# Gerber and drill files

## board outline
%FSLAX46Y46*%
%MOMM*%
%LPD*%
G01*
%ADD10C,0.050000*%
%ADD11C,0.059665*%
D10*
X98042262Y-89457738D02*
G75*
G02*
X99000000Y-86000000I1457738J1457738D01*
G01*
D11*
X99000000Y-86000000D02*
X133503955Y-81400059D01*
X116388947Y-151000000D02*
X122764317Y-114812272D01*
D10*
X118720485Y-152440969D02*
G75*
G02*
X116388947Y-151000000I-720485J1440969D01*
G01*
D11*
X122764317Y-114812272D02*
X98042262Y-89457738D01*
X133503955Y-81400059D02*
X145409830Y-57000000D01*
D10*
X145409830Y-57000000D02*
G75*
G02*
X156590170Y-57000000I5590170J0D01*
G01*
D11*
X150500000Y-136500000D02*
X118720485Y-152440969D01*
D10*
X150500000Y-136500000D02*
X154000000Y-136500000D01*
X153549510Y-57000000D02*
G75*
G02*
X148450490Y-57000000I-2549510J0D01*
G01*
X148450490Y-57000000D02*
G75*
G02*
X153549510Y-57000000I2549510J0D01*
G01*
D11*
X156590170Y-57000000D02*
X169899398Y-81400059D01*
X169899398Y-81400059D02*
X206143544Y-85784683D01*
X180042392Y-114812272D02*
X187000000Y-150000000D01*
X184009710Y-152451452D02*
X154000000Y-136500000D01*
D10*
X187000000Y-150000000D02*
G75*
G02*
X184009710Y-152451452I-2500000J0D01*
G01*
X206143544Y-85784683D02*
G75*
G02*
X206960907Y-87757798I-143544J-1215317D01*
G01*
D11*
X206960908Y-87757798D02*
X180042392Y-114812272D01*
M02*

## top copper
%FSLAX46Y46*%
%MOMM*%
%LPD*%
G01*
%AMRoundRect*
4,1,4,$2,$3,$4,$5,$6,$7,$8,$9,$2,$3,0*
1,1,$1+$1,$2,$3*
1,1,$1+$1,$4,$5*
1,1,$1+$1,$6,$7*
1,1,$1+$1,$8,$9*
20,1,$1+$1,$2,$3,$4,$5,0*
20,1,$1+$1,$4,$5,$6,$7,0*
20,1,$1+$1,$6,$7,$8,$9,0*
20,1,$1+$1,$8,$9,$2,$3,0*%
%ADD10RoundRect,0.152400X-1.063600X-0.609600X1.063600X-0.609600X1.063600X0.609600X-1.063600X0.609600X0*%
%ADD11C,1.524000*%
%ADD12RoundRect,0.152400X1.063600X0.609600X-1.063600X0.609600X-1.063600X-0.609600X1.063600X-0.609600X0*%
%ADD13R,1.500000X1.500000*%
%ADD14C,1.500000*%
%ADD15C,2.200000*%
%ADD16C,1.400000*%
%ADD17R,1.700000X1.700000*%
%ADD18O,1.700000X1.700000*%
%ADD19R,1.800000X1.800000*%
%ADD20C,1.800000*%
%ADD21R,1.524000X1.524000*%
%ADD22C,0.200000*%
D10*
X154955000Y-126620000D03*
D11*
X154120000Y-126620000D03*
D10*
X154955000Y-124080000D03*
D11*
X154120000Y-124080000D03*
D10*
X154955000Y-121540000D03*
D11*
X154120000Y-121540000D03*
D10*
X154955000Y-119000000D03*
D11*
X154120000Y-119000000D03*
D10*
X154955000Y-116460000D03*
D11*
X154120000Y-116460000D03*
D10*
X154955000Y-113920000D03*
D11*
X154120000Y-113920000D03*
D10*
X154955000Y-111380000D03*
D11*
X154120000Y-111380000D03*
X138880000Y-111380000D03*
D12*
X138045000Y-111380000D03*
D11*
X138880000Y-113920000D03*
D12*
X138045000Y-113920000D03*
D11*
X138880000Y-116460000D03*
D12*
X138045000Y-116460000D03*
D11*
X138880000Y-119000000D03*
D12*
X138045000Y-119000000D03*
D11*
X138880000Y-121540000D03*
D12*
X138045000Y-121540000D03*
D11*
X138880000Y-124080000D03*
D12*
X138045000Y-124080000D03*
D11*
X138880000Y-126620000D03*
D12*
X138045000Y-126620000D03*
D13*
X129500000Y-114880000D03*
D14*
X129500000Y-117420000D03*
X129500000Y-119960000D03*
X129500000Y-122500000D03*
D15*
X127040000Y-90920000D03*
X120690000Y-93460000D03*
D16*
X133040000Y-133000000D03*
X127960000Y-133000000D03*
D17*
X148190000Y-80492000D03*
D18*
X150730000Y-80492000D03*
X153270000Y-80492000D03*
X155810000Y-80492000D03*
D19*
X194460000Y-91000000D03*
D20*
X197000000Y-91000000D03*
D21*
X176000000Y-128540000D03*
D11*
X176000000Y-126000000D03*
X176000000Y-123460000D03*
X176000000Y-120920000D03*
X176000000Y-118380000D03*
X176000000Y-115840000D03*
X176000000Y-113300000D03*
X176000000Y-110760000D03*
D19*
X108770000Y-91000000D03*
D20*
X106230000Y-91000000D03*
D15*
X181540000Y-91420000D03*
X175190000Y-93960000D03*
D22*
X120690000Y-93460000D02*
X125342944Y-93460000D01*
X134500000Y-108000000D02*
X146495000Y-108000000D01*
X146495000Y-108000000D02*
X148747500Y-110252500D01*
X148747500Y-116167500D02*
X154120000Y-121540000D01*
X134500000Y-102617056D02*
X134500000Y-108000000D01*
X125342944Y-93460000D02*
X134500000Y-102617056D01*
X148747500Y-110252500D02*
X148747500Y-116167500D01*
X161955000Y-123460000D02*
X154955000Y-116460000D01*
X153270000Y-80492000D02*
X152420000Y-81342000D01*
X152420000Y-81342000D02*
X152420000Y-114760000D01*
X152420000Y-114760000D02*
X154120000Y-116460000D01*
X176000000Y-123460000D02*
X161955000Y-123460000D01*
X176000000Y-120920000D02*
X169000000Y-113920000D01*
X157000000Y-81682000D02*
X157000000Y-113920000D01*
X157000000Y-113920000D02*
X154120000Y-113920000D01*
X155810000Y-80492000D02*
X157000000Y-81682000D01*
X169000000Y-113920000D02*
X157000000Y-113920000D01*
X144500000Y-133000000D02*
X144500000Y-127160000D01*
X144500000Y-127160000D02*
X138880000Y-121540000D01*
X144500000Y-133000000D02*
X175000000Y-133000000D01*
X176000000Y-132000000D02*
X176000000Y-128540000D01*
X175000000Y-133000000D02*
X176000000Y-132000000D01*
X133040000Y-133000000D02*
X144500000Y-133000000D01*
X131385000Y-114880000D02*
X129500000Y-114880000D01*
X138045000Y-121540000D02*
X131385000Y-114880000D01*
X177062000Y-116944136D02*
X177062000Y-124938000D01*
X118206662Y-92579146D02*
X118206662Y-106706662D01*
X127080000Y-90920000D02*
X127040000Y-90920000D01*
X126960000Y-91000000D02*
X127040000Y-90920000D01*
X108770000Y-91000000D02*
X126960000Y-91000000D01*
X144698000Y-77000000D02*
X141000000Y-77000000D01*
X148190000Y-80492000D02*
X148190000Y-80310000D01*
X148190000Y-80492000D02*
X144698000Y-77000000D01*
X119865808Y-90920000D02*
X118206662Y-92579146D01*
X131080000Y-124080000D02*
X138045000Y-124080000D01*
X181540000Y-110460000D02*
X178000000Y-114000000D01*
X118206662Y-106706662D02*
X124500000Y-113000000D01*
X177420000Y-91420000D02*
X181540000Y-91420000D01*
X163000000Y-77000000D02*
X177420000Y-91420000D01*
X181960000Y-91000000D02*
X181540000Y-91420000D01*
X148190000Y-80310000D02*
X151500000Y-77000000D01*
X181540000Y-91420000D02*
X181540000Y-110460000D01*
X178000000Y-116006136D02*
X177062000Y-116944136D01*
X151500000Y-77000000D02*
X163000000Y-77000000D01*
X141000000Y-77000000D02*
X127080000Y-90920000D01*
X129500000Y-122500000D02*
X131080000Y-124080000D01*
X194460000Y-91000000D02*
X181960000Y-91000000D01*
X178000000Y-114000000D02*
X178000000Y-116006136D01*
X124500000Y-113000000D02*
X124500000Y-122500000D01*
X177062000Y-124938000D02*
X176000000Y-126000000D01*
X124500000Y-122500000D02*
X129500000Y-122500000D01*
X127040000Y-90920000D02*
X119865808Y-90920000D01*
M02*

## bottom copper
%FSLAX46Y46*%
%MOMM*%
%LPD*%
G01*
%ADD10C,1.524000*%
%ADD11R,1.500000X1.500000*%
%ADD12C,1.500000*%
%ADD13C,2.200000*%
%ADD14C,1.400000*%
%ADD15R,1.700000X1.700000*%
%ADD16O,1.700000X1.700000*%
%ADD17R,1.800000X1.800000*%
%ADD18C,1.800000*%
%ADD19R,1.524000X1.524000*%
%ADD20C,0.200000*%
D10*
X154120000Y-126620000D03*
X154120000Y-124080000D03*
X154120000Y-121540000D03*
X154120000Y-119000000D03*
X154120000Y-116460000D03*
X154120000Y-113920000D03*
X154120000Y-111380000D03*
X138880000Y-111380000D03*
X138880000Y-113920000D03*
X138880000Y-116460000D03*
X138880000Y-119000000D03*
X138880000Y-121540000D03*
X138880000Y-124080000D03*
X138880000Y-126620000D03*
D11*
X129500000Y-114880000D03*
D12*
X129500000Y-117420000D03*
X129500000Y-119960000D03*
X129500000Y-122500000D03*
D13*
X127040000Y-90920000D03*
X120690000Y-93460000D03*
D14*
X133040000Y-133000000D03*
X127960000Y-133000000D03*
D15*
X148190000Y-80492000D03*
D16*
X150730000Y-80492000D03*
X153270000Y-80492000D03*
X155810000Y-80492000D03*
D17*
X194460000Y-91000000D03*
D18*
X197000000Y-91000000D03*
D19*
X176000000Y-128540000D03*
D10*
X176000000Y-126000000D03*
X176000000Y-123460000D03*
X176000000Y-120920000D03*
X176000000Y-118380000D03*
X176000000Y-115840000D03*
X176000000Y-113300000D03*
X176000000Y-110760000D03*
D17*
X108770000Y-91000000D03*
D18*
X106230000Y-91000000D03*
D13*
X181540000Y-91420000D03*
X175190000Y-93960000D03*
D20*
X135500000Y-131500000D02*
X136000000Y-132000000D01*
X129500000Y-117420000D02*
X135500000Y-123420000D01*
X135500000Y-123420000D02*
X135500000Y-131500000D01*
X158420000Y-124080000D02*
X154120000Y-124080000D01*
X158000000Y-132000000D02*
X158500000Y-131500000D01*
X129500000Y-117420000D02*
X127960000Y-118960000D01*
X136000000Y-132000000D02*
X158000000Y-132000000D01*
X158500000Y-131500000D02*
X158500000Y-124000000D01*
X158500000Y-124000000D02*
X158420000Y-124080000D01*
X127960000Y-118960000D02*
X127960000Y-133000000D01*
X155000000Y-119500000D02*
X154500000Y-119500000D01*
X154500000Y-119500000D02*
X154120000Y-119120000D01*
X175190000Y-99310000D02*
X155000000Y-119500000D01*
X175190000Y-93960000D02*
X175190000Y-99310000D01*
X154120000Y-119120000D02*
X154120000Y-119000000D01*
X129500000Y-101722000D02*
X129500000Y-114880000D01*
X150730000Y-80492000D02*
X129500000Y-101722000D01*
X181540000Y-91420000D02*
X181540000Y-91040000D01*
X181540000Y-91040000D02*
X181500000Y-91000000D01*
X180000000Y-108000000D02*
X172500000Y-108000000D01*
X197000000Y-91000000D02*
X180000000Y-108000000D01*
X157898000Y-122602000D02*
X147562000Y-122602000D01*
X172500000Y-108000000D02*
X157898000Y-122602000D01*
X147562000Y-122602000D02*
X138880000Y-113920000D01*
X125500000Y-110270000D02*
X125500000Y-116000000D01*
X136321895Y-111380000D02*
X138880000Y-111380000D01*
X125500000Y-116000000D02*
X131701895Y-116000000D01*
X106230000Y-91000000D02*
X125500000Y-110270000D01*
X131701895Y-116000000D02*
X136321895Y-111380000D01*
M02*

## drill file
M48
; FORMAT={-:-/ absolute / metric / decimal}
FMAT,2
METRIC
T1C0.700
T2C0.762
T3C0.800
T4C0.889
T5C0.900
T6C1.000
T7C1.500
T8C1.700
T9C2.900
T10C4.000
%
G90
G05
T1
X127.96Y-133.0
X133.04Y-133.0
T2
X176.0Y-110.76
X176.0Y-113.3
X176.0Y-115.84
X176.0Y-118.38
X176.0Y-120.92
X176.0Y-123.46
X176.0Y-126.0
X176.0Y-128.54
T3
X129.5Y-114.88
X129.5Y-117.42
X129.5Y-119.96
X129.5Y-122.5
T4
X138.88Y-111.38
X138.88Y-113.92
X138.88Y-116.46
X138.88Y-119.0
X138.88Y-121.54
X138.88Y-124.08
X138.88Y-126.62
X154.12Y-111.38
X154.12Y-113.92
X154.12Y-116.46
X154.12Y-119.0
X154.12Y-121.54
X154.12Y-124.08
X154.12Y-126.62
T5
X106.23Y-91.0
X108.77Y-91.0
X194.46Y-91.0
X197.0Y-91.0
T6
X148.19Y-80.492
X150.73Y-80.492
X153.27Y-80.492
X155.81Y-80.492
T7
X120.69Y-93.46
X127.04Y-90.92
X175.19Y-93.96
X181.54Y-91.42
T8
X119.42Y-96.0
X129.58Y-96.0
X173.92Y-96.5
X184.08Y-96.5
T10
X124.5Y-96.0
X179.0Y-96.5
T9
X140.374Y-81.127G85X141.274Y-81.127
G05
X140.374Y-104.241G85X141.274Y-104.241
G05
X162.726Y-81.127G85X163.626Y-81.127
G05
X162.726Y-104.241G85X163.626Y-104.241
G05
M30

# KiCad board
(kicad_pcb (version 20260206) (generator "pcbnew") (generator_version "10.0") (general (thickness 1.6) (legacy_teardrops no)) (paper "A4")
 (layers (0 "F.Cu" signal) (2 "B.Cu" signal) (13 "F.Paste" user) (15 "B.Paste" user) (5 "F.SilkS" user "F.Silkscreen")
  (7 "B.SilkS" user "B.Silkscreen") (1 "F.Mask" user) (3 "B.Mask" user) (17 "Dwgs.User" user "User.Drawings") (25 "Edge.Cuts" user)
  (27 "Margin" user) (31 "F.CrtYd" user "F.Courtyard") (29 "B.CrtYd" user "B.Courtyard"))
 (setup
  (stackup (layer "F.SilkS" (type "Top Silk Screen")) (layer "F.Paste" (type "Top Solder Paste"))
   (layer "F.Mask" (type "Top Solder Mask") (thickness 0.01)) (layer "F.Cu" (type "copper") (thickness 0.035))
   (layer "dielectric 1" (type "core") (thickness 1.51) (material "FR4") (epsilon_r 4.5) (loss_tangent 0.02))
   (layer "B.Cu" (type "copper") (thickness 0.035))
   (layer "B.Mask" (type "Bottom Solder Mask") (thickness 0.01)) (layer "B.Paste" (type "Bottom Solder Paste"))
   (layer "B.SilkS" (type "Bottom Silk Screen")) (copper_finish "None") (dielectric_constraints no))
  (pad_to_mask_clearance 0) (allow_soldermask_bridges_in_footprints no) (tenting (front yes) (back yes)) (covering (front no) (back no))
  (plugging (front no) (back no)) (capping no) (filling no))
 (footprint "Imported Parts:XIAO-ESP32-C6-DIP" (layer "F.Cu") (at 146.5 119 -90)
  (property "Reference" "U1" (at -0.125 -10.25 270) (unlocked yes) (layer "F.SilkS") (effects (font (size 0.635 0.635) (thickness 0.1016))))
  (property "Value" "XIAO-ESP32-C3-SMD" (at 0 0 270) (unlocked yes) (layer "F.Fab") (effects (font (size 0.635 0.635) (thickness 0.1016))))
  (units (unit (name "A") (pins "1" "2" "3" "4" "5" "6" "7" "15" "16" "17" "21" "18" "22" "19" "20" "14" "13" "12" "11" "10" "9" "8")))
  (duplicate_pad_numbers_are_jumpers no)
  (pad "1" smd roundrect (at 7.62 -8.455) (size 2.432 1.524) (layers "F.Cu" "F.Mask") (roundrect_rratio 0.1)
   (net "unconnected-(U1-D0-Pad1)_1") (thermal_bridge_angle 45))
  (pad "1" thru_hole circle (at 7.62 -7.62) (size 1.524 1.524) (drill 0.889) (layers "*.Cu" "*.Mask") (remove_unused_layers no)
   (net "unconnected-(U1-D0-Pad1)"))
  (pad "2" smd roundrect (at 5.08 -8.455) (size 2.432 1.524) (layers "F.Cu" "F.Mask") (roundrect_rratio 0.1) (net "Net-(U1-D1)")
   (thermal_bridge_angle 45))
  (pad "2" thru_hole circle (at 5.08 -7.62) (size 1.524 1.524) (drill 0.889) (layers "*.Cu" "*.Mask") (remove_unused_layers no)
   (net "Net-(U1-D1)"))
  (pad "3" smd roundrect (at 2.54 -8.455) (size 2.432 1.524) (layers "F.Cu" "F.Mask") (roundrect_rratio 0.1) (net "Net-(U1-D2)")
   (thermal_bridge_angle 45))
  (pad "3" thru_hole circle (at 2.54 -7.62) (size 1.524 1.524) (drill 0.889) (layers "*.Cu" "*.Mask") (remove_unused_layers no)
   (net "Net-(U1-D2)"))
  (pad "4" smd roundrect (at 0 -8.455) (size 2.432 1.524) (layers "F.Cu" "F.Mask") (roundrect_rratio 0.1) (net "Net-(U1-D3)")
   (thermal_bridge_angle 45))
  (pad "4" thru_hole circle (at 0 -7.62) (size 1.524 1.524) (drill 0.889) (layers "*.Cu" "*.Mask") (remove_unused_layers no)
   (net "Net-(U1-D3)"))
  (pad "5" smd roundrect (at -2.54 -8.455) (size 2.432 1.524) (layers "F.Cu" "F.Mask") (roundrect_rratio 0.1) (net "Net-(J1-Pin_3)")
   (thermal_bridge_angle 45))
  (pad "5" thru_hole circle (at -2.54 -7.62) (size 1.524 1.524) (drill 0.889) (layers "*.Cu" "*.Mask") (remove_unused_layers no)
   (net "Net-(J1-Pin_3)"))
  (pad "6" smd roundrect (at -5.08 -8.455) (size 2.432 1.524) (layers "F.Cu" "F.Mask") (roundrect_rratio 0.1) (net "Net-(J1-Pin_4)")
   (thermal_bridge_angle 45))
  (pad "6" thru_hole circle (at -5.08 -7.62) (size 1.524 1.524) (drill 0.889) (layers "*.Cu" "*.Mask") (remove_unused_layers no)
   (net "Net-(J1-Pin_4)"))
  (pad "7" smd roundrect (at -7.62 -8.455) (size 2.432 1.524) (layers "F.Cu" "F.Mask") (roundrect_rratio 0.1)
   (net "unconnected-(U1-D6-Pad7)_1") (thermal_bridge_angle 45))
  (pad "7" thru_hole circle (at -7.62 -7.62) (size 1.524 1.524) (drill 0.889) (layers "*.Cu" "*.Mask") (remove_unused_layers no)
   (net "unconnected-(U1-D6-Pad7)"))
  (pad "8" thru_hole circle (at -7.62 7.62 180) (size 1.524 1.524) (drill 0.889) (layers "*.Cu" "*.Mask") (remove_unused_layers no)
   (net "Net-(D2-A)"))
  (pad "8" smd roundrect (at -7.62 8.455 180) (size 2.432 1.524) (layers "F.Cu" "F.Mask") (roundrect_rratio 0.1) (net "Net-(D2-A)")
   (thermal_bridge_angle 45))
  (pad "9" thru_hole circle (at -5.08 7.62 180) (size 1.524 1.524) (drill 0.889) (layers "*.Cu" "*.Mask") (remove_unused_layers no)
   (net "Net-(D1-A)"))
  (pad "9" smd roundrect (at -5.08 8.455 180) (size 2.432 1.524) (layers "F.Cu" "F.Mask") (roundrect_rratio 0.1) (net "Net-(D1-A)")
   (thermal_bridge_angle 45))
  (pad "10" thru_hole circle (at -2.54 7.62 180) (size 1.524 1.524) (drill 0.889) (layers "*.Cu" "*.Mask") (remove_unused_layers no)
   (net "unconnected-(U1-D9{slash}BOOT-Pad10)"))
  (pad "10" smd roundrect (at -2.54 8.455 180) (size 2.432 1.524) (layers "F.Cu" "F.Mask") (roundrect_rratio 0.1)
   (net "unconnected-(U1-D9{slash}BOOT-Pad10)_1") (thermal_bridge_angle 45))
  (pad "11" thru_hole circle (at 0 7.62 180) (size 1.524 1.524) (drill 0.889) (layers "*.Cu" "*.Mask") (remove_unused_layers no)
   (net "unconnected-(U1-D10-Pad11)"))
  (pad "11" smd roundrect (at 0 8.455 180) (size 2.432 1.524) (layers "F.Cu" "F.Mask") (roundrect_rratio 0.1)
   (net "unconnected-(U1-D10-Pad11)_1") (thermal_bridge_angle 45))
  (pad "12" thru_hole circle (at 2.54 7.62 180) (size 1.524 1.524) (drill 0.889) (layers "*.Cu" "*.Mask") (remove_unused_layers no)
   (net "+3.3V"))
  (pad "12" smd roundrect (at 2.54 8.455 180) (size 2.432 1.524) (layers "F.Cu" "F.Mask") (roundrect_rratio 0.1) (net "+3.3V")
   (thermal_bridge_angle 45))
  (pad "13" thru_hole circle (at 5.08 7.62 180) (size 1.524 1.524) (drill 0.889) (layers "*.Cu" "*.Mask") (remove_unused_layers no)
   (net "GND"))
  (pad "13" smd roundrect (at 5.08 8.455 180) (size 2.432 1.524) (layers "F.Cu" "F.Mask") (roundrect_rratio 0.1) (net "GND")
   (thermal_bridge_angle 45))
  (pad "14" thru_hole circle (at 7.62 7.62 180) (size 1.524 1.524) (drill 0.889) (layers "*.Cu" "*.Mask") (remove_unused_layers no)
   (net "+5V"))
  (pad "14" smd roundrect (at 7.62 8.455 180) (size 2.432 1.524) (layers "F.Cu" "F.Mask") (roundrect_rratio 0.1) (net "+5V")
   (thermal_bridge_angle 45)))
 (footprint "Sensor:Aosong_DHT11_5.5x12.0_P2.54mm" (layer "F.Cu") (at 129.5 114.88)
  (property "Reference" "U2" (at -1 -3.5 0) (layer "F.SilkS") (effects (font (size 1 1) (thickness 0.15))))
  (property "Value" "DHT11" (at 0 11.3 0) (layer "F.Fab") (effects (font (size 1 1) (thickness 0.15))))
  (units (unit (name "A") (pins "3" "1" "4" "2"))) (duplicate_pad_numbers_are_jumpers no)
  (pad "1" thru_hole rect (at 0 0) (size 1.5 1.5) (drill 0.8) (layers "*.Cu" "*.Mask") (remove_unused_layers no) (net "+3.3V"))
  (pad "2" thru_hole circle (at 0 2.54) (size 1.5 1.5) (drill 0.8) (layers "*.Cu" "*.Mask") (remove_unused_layers no) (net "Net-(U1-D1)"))
  (pad "3" thru_hole circle (at 0 5.08) (size 1.5 1.5) (drill 0.8) (layers "*.Cu" "*.Mask") (remove_unused_layers no)
   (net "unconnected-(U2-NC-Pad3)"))
  (pad "4" thru_hole circle (at 0 7.62) (size 1.5 1.5) (drill 0.8) (layers "*.Cu" "*.Mask") (remove_unused_layers no) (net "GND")))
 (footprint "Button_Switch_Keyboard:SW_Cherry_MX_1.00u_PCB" (layer "F.Cu") (at 127.04 90.92)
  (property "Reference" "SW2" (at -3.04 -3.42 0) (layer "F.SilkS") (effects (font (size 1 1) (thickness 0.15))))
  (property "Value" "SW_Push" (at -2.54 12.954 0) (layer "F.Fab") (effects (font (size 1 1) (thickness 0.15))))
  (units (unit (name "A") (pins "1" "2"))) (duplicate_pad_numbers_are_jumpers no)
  (pad "" np_thru_hole circle (at -7.62 5.08) (size 1.7 1.7) (drill 1.7) (layers "*.Cu" "*.Mask"))
  (pad "" np_thru_hole circle (at -2.54 5.08) (size 4 4) (drill 4) (layers "*.Cu" "*.Mask"))
  (pad "" np_thru_hole circle (at 2.54 5.08) (size 1.7 1.7) (drill 1.7) (layers "*.Cu" "*.Mask"))
  (pad "1" thru_hole circle (at 0 0) (size 2.2 2.2) (drill 1.5) (layers "*.Cu" "*.Mask") (remove_unused_layers no) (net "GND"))
  (pad "2" thru_hole circle (at -6.35 2.54) (size 2.2 2.2) (drill 1.5) (layers "*.Cu" "*.Mask") (remove_unused_layers no)
   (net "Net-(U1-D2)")))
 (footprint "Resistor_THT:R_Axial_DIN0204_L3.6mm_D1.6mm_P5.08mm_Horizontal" (layer "F.Cu") (at 133.04 133 180)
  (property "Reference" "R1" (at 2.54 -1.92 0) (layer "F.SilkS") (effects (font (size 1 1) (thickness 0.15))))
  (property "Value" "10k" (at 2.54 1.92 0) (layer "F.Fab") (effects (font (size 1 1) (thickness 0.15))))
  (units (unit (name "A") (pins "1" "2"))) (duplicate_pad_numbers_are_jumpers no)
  (pad "1" thru_hole circle (at 0 0 180) (size 1.4 1.4) (drill 0.7) (layers "*.Cu" "*.Mask") (remove_unused_layers no) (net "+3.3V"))
  (pad "2" thru_hole circle (at 5.08 0 180) (size 1.4 1.4) (drill 0.7) (layers "*.Cu" "*.Mask") (remove_unused_layers no)
   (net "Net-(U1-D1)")))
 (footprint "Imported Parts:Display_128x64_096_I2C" (layer "F.Cu") (at 152 80.492)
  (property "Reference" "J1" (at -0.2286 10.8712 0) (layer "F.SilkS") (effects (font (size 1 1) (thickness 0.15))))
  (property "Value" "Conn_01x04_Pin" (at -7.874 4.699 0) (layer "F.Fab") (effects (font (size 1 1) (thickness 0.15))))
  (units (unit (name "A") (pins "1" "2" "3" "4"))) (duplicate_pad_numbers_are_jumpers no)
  (pad "" np_thru_hole oval (at -11.176 0.635) (size 3.8 2.9) (drill oval 3.8 2.9) (layers "*.Cu" "*.Mask"))
  (pad "" np_thru_hole oval (at -11.176 23.749) (size 3.8 2.9) (drill oval 3.8 2.9) (layers "*.Cu" "*.Mask"))
  (pad "" np_thru_hole oval (at 11.176 0.635) (size 3.8 2.9) (drill oval 3.8 2.9) (layers "*.Cu" "*.Mask"))
  (pad "" np_thru_hole oval (at 11.176 23.749) (size 3.8 2.9) (drill oval 3.8 2.9) (layers "*.Cu" "*.Mask"))
  (pad "1" thru_hole rect (at -3.81 0 90) (size 1.7 1.7) (drill 1) (layers "*.Cu" "*.Mask") (remove_unused_layers no) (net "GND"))
  (pad "2" thru_hole oval (at -1.27 0 90) (size 1.7 1.7) (drill 1) (layers "*.Cu" "*.Mask") (remove_unused_layers no) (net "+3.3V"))
  (pad "3" thru_hole oval (at 1.27 0 90) (size 1.7 1.7) (drill 1) (layers "*.Cu" "*.Mask") (remove_unused_layers no) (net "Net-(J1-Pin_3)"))
  (pad "4" thru_hole oval (at 3.81 0 90) (size 1.7 1.7) (drill 1) (layers "*.Cu" "*.Mask") (remove_unused_layers no) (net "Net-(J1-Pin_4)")))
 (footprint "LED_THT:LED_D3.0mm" (layer "F.Cu") (at 194.46 91)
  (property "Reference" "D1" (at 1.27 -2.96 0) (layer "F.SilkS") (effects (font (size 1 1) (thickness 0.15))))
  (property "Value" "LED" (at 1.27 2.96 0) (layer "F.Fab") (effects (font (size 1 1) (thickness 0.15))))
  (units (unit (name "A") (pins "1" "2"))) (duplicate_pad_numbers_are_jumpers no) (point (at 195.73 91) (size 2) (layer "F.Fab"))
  (pad "1" thru_hole rect (at 0 0) (size 1.8 1.8) (drill 0.9) (layers "*.Cu" "*.Mask") (remove_unused_layers no) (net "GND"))
  (pad "2" thru_hole circle (at 2.54 0) (size 1.8 1.8) (drill 0.9) (layers "*.Cu" "*.Mask") (remove_unused_layers no) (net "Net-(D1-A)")))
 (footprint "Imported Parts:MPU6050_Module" (layer "F.Cu") (at 176 128.54 180)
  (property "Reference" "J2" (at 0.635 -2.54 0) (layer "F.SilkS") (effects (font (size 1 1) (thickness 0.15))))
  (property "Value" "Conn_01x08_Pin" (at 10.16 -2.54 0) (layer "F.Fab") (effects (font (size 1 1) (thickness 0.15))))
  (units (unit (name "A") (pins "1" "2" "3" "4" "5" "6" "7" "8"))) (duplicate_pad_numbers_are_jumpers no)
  (pad "1" thru_hole rect (at 0 0 180) (size 1.524 1.524) (drill 0.762) (layers "*.Cu" "*.Mask") (remove_unused_layers no) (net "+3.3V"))
  (pad "2" thru_hole circle (at 0 2.54 180) (size 1.524 1.524) (drill 0.762) (layers "*.Cu" "*.Mask") (remove_unused_layers no) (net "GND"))
  (pad "3" thru_hole circle (at 0 5.08 180) (size 1.524 1.524) (drill 0.762) (layers "*.Cu" "*.Mask") (remove_unused_layers no)
   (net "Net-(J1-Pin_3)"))
  (pad "4" thru_hole circle (at 0 7.62 180) (size 1.524 1.524) (drill 0.762) (layers "*.Cu" "*.Mask") (remove_unused_layers no)
   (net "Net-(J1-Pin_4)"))
  (pad "5" thru_hole circle (at 0 10.16 180) (size 1.524 1.524) (drill 0.762) (layers "*.Cu" "*.Mask") (remove_unused_layers no)
   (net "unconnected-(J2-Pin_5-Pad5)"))
  (pad "6" thru_hole circle (at 0 12.7 180) (size 1.524 1.524) (drill 0.762) (layers "*.Cu" "*.Mask") (remove_unused_layers no)
   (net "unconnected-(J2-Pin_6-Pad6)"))
  (pad "7" thru_hole circle (at 0 15.24 180) (size 1.524 1.524) (drill 0.762) (layers "*.Cu" "*.Mask") (remove_unused_layers no)
   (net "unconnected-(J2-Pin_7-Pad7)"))
  (pad "8" thru_hole circle (at 0 17.78 180) (size 1.524 1.524) (drill 0.762) (layers "*.Cu" "*.Mask") (remove_unused_layers no)
   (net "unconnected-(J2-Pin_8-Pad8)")))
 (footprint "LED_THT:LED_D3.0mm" (layer "F.Cu") (at 108.77 91 180)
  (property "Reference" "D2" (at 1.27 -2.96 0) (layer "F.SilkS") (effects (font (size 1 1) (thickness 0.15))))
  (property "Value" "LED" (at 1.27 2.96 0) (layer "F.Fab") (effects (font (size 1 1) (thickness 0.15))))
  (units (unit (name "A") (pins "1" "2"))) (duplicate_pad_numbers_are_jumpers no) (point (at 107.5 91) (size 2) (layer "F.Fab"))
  (pad "1" thru_hole rect (at 0 0 180) (size 1.8 1.8) (drill 0.9) (layers "*.Cu" "*.Mask") (remove_unused_layers no) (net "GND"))
  (pad "2" thru_hole circle (at 2.54 0 180) (size 1.8 1.8) (drill 0.9) (layers "*.Cu" "*.Mask") (remove_unused_layers no) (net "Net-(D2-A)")))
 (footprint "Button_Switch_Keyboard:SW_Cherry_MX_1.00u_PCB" (layer "F.Cu") (at 181.54 91.42)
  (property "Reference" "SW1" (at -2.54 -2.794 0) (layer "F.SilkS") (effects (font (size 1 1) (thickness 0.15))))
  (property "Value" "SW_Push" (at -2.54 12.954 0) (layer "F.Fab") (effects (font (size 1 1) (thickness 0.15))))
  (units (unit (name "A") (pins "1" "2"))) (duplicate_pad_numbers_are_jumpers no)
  (pad "" np_thru_hole circle (at -7.62 5.08) (size 1.7 1.7) (drill 1.7) (layers "*.Cu" "*.Mask"))
  (pad "" np_thru_hole circle (at -2.54 5.08) (size 4 4) (drill 4) (layers "*.Cu" "*.Mask"))
  (pad "" np_thru_hole circle (at 2.54 5.08) (size 1.7 1.7) (drill 1.7) (layers "*.Cu" "*.Mask"))
  (pad "1" thru_hole circle (at 0 0) (size 2.2 2.2) (drill 1.5) (layers "*.Cu" "*.Mask") (remove_unused_layers no) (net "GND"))
  (pad "2" thru_hole circle (at -6.35 2.54) (size 2.2 2.2) (drill 1.5) (layers "*.Cu" "*.Mask") (remove_unused_layers no)
   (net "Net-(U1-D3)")))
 (gr_arc (start 98.042262 89.457738) (mid 97.513251 87.449702) (end 99 86) (stroke (width 0.05) (type default)) (layer "Edge.Cuts"))
 (gr_line (start 99 86) (end 133.503955 81.400059) (stroke (width 0.059665) (type default)) (layer "Edge.Cuts"))
 (gr_line (start 116.388947 151) (end 122.764317 114.812272) (stroke (width 0.059665) (type default)) (layer "Edge.Cuts"))
 (gr_arc (start 118.720485 152.440969) (mid 117.15302 152.370443) (end 116.388947 151) (stroke (width 0.05) (type default))
  (layer "Edge.Cuts"))
 (gr_line (start 122.764317 114.812272) (end 98.042262 89.457738) (stroke (width 0.059665) (type default)) (layer "Edge.Cuts"))
 (gr_line (start 133.503955 81.400059) (end 145.40983 57) (stroke (width 0.059665) (type default)) (layer "Edge.Cuts"))
 (gr_arc (start 145.40983 57) (mid 151 51.40983) (end 156.59017 57) (stroke (width 0.05) (type default)) (layer "Edge.Cuts"))
 (gr_line (start 150.5 136.5) (end 118.720485 152.440969) (stroke (width 0.059665) (type default)) (layer "Edge.Cuts"))
 (gr_line (start 150.5 136.5) (end 154 136.5) (stroke (width 0.05) (type default)) (layer "Edge.Cuts"))
 (gr_circle (center 151 57) (end 151.5 54.5) (stroke (width 0.05) (type default)) (fill no) (layer "Edge.Cuts"))
 (gr_line (start 156.59017 57) (end 169.899398 81.400059) (stroke (width 0.059665) (type default)) (layer "Edge.Cuts"))
 (gr_line (start 169.899398 81.400059) (end 206.143544 85.784683) (stroke (width 0.059665) (type default)) (layer "Edge.Cuts"))
 (gr_line (start 180.042392 114.812272) (end 187 150) (stroke (width 0.059665) (type default)) (layer "Edge.Cuts"))
 (gr_line (start 184.00971 152.451452) (end 154 136.5) (stroke (width 0.059665) (type default)) (layer "Edge.Cuts"))
 (gr_arc (start 187 150) (mid 186.084972 151.933355) (end 184.00971 152.451452) (stroke (width 0.05) (type default)) (layer "Edge.Cuts"))
 (gr_arc (start 206.143544 85.784683) (mid 207.130597 86.53165) (end 206.960908 87.757798) (stroke (width 0.05) (type default))
  (layer "Edge.Cuts"))
 (gr_line (start 206.960908 87.757798) (end 180.042392 114.812272) (stroke (width 0.059665) (type default)) (layer "Edge.Cuts"))
 (segment (start 135.5 131.5) (end 136 132) (width 0.2) (layer "B.Cu") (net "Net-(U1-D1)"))
 (segment (start 129.5 117.42) (end 135.5 123.42) (width 0.2) (layer "B.Cu") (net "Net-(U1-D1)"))
 (segment (start 135.5 123.42) (end 135.5 131.5) (width 0.2) (layer "B.Cu") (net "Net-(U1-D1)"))
 (segment (start 158.42 124.08) (end 154.12 124.08) (width 0.2) (layer "B.Cu") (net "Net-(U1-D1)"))
 (segment (start 158 132) (end 158.5 131.5) (width 0.2) (layer "B.Cu") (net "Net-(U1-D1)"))
 (segment (start 129.5 117.42) (end 127.96 118.96) (width 0.2) (layer "B.Cu") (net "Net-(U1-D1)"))
 (segment (start 136 132) (end 158 132) (width 0.2) (layer "B.Cu") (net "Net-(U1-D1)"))
 (segment (start 158.5 131.5) (end 158.5 124) (width 0.2) (layer "B.Cu") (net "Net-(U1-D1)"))
 (segment (start 158.5 124) (end 158.42 124.08) (width 0.2) (layer "B.Cu") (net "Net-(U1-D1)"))
 (segment (start 127.96 118.96) (end 127.96 133) (width 0.2) (layer "B.Cu") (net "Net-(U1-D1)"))
 (segment (start 120.69 93.46) (end 125.342944 93.46) (width 0.2) (layer "F.Cu") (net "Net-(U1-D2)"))
 (segment (start 134.5 108) (end 146.495 108) (width 0.2) (layer "F.Cu") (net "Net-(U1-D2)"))
 (segment (start 146.495 108) (end 148.7475 110.2525) (width 0.2) (layer "F.Cu") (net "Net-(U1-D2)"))
 (segment (start 148.7475 116.1675) (end 154.12 121.54) (width 0.2) (layer "F.Cu") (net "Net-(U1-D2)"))
 (segment (start 134.5 102.617056) (end 134.5 108) (width 0.2) (layer "F.Cu") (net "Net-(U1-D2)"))
 (segment (start 125.342944 93.46) (end 134.5 102.617056) (width 0.2) (layer "F.Cu") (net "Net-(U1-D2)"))
 (segment (start 148.7475 110.2525) (end 148.7475 116.1675) (width 0.2) (layer "F.Cu") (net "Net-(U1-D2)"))
 (segment (start 155 119.5) (end 154.5 119.5) (width 0.2) (layer "B.Cu") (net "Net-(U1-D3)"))
 (segment (start 154.5 119.5) (end 154.12 119.12) (width 0.2) (layer "B.Cu") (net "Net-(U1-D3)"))
 (segment (start 175.19 99.31) (end 155 119.5) (width 0.2) (layer "B.Cu") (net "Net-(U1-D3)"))
 (segment (start 175.19 93.96) (end 175.19 99.31) (width 0.2) (layer "B.Cu") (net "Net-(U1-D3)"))
 (segment (start 154.12 119.12) (end 154.12 119) (width 0.2) (layer "B.Cu") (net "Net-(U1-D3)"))
 (segment (start 161.955 123.46) (end 154.955 116.46) (width 0.2) (layer "F.Cu") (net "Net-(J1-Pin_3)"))
 (segment (start 153.27 80.492) (end 152.42 81.342) (width 0.2) (layer "F.Cu") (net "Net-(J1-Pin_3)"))
 (segment (start 152.42 81.342) (end 152.42 114.76) (width 0.2) (layer "F.Cu") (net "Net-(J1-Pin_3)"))
 (segment (start 152.42 114.76) (end 154.12 116.46) (width 0.2) (layer "F.Cu") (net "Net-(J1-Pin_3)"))
 (segment (start 176 123.46) (end 161.955 123.46) (width 0.2) (layer "F.Cu") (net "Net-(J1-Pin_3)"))
 (segment (start 176 120.92) (end 169 113.92) (width 0.2) (layer "F.Cu") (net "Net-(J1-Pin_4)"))
 (segment (start 157 81.682) (end 157 113.92) (width 0.2) (layer "F.Cu") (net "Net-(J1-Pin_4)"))
 (segment (start 157 113.92) (end 154.12 113.92) (width 0.2) (layer "F.Cu") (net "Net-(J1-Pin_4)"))
 (segment (start 155.81 80.492) (end 157 81.682) (width 0.2) (layer "F.Cu") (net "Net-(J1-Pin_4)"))
 (segment (start 169 113.92) (end 157 113.92) (width 0.2) (layer "F.Cu") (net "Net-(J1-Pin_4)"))
 (segment (start 144.5 133) (end 144.5 127.16) (width 0.2) (layer "F.Cu") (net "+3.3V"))
 (segment (start 144.5 127.16) (end 138.88 121.54) (width 0.2) (layer "F.Cu") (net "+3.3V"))
 (segment (start 144.5 133) (end 175 133) (width 0.2) (layer "F.Cu") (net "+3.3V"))
 (segment (start 176 132) (end 176 128.54) (width 0.2) (layer "F.Cu") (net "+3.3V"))
 (segment (start 175 133) (end 176 132) (width 0.2) (layer "F.Cu") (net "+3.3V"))
 (segment (start 133.04 133) (end 144.5 133) (width 0.2) (layer "F.Cu") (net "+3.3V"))
 (segment (start 131.385 114.88) (end 129.5 114.88) (width 0.2) (layer "F.Cu") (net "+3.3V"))
 (segment (start 138.045 121.54) (end 131.385 114.88) (width 0.2) (layer "F.Cu") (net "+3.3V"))
 (segment (start 129.5 101.722) (end 129.5 114.88) (width 0.2) (layer "B.Cu") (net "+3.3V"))
 (segment (start 150.73 80.492) (end 129.5 101.722) (width 0.2) (layer "B.Cu") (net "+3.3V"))
 (segment (start 177.062 116.944136) (end 177.062 124.938) (width 0.2) (layer "F.Cu") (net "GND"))
 (segment (start 118.206662 92.579146) (end 118.206662 106.706662) (width 0.2) (layer "F.Cu") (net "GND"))
 (segment (start 127.08 90.92) (end 127.04 90.92) (width 0.2) (layer "F.Cu") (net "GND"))
 (segment (start 126.96 91) (end 127.04 90.92) (width 0.2) (layer "F.Cu") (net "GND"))
 (segment (start 108.77 91) (end 126.96 91) (width 0.2) (layer "F.Cu") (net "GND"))
 (segment (start 144.698 77) (end 141 77) (width 0.2) (layer "F.Cu") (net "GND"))
 (segment (start 148.19 80.492) (end 148.19 80.31) (width 0.2) (layer "F.Cu") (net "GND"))
 (segment (start 148.19 80.492) (end 144.698 77) (width 0.2) (layer "F.Cu") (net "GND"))
 (segment (start 119.865808 90.92) (end 118.206662 92.579146) (width 0.2) (layer "F.Cu") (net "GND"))
 (segment (start 131.08 124.08) (end 138.045 124.08) (width 0.2) (layer "F.Cu") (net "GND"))
 (segment (start 181.54 110.46) (end 178 114) (width 0.2) (layer "F.Cu") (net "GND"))
 (segment (start 118.206662 106.706662) (end 124.5 113) (width 0.2) (layer "F.Cu") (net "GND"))
 (segment (start 177.42 91.42) (end 181.54 91.42) (width 0.2) (layer "F.Cu") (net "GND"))
 (segment (start 163 77) (end 177.42 91.42) (width 0.2) (layer "F.Cu") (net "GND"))
 (segment (start 181.96 91) (end 181.54 91.42) (width 0.2) (layer "F.Cu") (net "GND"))
 (segment (start 148.19 80.31) (end 151.5 77) (width 0.2) (layer "F.Cu") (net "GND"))
 (segment (start 181.54 91.42) (end 181.54 110.46) (width 0.2) (layer "F.Cu") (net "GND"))
 (segment (start 178 116.006136) (end 177.062 116.944136) (width 0.2) (layer "F.Cu") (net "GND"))
 (segment (start 151.5 77) (end 163 77) (width 0.2) (layer "F.Cu") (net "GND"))
 (segment (start 141 77) (end 127.08 90.92) (width 0.2) (layer "F.Cu") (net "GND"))
 (segment (start 129.5 122.5) (end 131.08 124.08) (width 0.2) (layer "F.Cu") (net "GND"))
 (segment (start 194.46 91) (end 181.96 91) (width 0.2) (layer "F.Cu") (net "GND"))
 (segment (start 178 114) (end 178 116.006136) (width 0.2) (layer "F.Cu") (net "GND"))
 (segment (start 124.5 113) (end 124.5 122.5) (width 0.2) (layer "F.Cu") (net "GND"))
 (segment (start 177.062 124.938) (end 176 126) (width 0.2) (layer "F.Cu") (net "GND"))
 (segment (start 124.5 122.5) (end 129.5 122.5) (width 0.2) (layer "F.Cu") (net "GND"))
 (segment (start 127.04 90.92) (end 119.865808 90.92) (width 0.2) (layer "F.Cu") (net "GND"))
 (segment (start 181.54 91.42) (end 181.54 91.04) (width 0.2) (layer "B.Cu") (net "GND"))
 (segment (start 181.54 91.04) (end 181.5 91) (width 0.2) (layer "B.Cu") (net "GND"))
 (segment (start 180 108) (end 172.5 108) (width 0.2) (layer "B.Cu") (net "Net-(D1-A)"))
 (segment (start 197 91) (end 180 108) (width 0.2) (layer "B.Cu") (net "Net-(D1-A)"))
 (segment (start 157.898 122.602) (end 147.562 122.602) (width 0.2) (layer "B.Cu") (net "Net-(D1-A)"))
 (segment (start 172.5 108) (end 157.898 122.602) (width 0.2) (layer "B.Cu") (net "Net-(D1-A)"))
 (segment (start 147.562 122.602) (end 138.88 113.92) (width 0.2) (layer "B.Cu") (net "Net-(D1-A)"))
 (segment (start 125.5 110.27) (end 125.5 116) (width 0.2) (layer "B.Cu") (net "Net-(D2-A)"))
 (segment (start 136.321895 111.38) (end 138.88 111.38) (width 0.2) (layer "B.Cu") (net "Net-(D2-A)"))
 (segment (start 125.5 116) (end 131.701895 116) (width 0.2) (layer "B.Cu") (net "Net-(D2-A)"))
 (segment (start 106.23 91) (end 125.5 110.27) (width 0.2) (layer "B.Cu") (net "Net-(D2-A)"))
 (segment (start 131.701895 116) (end 136.321895 111.38) (width 0.2) (layer "B.Cu") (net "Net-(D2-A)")))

